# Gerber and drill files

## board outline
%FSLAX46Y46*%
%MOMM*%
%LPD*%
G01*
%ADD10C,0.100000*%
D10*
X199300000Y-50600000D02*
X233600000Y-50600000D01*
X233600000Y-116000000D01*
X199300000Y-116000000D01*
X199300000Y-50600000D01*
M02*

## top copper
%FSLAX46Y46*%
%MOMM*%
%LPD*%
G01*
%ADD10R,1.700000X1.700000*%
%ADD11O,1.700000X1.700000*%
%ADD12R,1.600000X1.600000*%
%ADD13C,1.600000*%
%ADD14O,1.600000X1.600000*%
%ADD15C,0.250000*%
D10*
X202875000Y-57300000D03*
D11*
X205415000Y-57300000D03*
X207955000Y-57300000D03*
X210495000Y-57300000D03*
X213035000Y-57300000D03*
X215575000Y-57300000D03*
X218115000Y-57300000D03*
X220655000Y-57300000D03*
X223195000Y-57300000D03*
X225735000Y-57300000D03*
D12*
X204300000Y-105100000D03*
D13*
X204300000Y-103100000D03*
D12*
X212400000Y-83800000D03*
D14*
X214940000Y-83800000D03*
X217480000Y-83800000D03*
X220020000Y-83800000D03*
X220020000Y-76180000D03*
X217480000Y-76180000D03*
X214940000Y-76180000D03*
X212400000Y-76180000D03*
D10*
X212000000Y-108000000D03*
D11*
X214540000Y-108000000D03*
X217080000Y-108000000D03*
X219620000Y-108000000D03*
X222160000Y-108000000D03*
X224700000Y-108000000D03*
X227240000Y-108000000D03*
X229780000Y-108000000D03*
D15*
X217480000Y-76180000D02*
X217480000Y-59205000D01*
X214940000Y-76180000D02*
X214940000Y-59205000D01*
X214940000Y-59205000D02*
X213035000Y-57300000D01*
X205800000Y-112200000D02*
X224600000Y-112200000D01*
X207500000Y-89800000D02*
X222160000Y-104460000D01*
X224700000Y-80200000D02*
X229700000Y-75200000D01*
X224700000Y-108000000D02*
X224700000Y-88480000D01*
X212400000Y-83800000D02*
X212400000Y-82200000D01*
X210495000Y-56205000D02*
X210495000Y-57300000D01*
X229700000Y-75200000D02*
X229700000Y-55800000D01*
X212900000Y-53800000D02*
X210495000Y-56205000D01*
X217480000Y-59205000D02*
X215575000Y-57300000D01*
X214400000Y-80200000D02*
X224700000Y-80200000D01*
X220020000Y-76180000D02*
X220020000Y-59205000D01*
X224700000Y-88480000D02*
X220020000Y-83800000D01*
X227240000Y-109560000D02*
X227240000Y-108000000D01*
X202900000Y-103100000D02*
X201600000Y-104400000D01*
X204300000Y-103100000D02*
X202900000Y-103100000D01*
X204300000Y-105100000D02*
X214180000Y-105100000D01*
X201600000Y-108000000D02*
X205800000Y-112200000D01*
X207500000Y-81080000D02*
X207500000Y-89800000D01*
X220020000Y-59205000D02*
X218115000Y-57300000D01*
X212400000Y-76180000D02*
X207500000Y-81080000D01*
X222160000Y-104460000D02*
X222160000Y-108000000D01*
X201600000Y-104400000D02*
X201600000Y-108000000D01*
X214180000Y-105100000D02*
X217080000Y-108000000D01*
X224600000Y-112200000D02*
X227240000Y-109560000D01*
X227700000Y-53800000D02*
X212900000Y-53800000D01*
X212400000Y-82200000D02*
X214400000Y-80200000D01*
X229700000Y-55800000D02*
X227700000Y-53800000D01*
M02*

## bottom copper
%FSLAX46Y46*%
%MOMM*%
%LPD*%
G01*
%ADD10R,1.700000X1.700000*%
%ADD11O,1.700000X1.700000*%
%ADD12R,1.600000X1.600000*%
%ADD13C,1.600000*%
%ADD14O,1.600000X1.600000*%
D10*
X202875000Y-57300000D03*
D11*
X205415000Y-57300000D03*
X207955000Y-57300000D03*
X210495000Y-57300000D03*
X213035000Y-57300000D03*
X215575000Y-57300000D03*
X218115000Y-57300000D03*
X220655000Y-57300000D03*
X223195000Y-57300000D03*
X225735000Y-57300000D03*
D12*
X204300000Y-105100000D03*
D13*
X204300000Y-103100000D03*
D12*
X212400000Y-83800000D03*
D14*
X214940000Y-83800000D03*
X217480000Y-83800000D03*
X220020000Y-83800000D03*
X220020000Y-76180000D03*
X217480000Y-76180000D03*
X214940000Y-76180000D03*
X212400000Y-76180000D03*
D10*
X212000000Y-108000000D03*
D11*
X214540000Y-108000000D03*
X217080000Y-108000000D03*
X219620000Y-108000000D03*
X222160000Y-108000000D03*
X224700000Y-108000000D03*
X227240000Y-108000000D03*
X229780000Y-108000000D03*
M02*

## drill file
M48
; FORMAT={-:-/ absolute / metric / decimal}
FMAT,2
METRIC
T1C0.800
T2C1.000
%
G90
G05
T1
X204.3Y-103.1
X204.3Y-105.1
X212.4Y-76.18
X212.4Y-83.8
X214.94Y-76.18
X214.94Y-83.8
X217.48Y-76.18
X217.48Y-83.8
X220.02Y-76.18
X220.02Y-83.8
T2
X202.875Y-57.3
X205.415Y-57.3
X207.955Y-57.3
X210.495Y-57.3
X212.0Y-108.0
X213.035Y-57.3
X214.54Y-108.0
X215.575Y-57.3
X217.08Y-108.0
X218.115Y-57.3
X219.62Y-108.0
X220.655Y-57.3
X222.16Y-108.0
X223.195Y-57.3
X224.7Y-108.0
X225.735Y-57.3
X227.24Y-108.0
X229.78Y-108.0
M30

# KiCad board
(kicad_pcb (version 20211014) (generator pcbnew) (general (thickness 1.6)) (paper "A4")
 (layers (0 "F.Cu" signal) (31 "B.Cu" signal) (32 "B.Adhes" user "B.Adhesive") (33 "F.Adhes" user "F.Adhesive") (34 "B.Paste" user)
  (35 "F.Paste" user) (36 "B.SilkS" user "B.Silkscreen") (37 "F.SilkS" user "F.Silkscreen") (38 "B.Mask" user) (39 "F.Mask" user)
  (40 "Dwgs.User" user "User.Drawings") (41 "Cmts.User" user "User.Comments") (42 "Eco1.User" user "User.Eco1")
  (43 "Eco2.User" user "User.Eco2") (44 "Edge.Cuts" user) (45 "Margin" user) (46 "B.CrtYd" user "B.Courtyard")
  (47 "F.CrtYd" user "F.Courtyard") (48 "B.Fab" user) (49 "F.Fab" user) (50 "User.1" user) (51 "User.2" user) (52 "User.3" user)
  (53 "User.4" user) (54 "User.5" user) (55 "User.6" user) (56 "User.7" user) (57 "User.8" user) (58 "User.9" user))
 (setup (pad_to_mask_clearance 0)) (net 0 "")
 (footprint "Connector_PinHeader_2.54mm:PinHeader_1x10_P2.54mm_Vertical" (layer "F.Cu") (at 202.875 57.3 90)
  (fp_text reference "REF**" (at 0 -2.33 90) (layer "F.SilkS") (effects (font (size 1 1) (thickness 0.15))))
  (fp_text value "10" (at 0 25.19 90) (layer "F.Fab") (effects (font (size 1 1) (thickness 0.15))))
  (pad "1" thru_hole rect (at 0 0 90) (size 1.7 1.7) (drill 1) (layers *.Cu *.Mask))
  (pad "2" thru_hole oval (at 0 2.54 90) (size 1.7 1.7) (drill 1) (layers *.Cu *.Mask))
  (pad "3" thru_hole oval (at 0 5.08 90) (size 1.7 1.7) (drill 1) (layers *.Cu *.Mask))
  (pad "4" thru_hole oval (at 0 7.62 90) (size 1.7 1.7) (drill 1) (layers *.Cu *.Mask))
  (pad "5" thru_hole oval (at 0 10.16 90) (size 1.7 1.7) (drill 1) (layers *.Cu *.Mask))
  (pad "6" thru_hole oval (at 0 12.7 90) (size 1.7 1.7) (drill 1) (layers *.Cu *.Mask))
  (pad "7" thru_hole oval (at 0 15.24 90) (size 1.7 1.7) (drill 1) (layers *.Cu *.Mask))
  (pad "8" thru_hole oval (at 0 17.78 90) (size 1.7 1.7) (drill 1) (layers *.Cu *.Mask))
  (pad "9" thru_hole oval (at 0 20.32 90) (size 1.7 1.7) (drill 1) (layers *.Cu *.Mask))
  (pad "10" thru_hole oval (at 0 22.86 90) (size 1.7 1.7) (drill 1) (layers *.Cu *.Mask)))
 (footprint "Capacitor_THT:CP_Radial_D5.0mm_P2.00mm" (layer "F.Cu") (at 204.3 105.1 90)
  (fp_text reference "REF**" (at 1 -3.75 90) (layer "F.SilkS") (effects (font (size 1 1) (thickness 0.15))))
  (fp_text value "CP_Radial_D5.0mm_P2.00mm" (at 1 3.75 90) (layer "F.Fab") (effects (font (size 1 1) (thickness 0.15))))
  (pad "1" thru_hole rect (at 0 0 90) (size 1.6 1.6) (drill 0.8) (layers *.Cu *.Mask))
  (pad "2" thru_hole circle (at 2 0 90) (size 1.6 1.6) (drill 0.8) (layers *.Cu *.Mask)))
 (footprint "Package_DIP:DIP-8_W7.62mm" (layer "F.Cu") (at 212.4 83.8 90)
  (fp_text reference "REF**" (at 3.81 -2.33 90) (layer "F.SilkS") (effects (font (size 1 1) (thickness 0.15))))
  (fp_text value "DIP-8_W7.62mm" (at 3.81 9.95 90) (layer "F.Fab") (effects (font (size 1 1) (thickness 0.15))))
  (pad "1" thru_hole rect (at 0 0 90) (size 1.6 1.6) (drill 0.8) (layers *.Cu *.Mask))
  (pad "2" thru_hole oval (at 0 2.54 90) (size 1.6 1.6) (drill 0.8) (layers *.Cu *.Mask))
  (pad "3" thru_hole oval (at 0 5.08 90) (size 1.6 1.6) (drill 0.8) (layers *.Cu *.Mask))
  (pad "4" thru_hole oval (at 0 7.62 90) (size 1.6 1.6) (drill 0.8) (layers *.Cu *.Mask))
  (pad "5" thru_hole oval (at 7.62 7.62 90) (size 1.6 1.6) (drill 0.8) (layers *.Cu *.Mask))
  (pad "6" thru_hole oval (at 7.62 5.08 90) (size 1.6 1.6) (drill 0.8) (layers *.Cu *.Mask))
  (pad "7" thru_hole oval (at 7.62 2.54 90) (size 1.6 1.6) (drill 0.8) (layers *.Cu *.Mask))
  (pad "8" thru_hole oval (at 7.62 0 90) (size 1.6 1.6) (drill 0.8) (layers *.Cu *.Mask)))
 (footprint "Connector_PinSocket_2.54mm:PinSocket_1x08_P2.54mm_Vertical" (layer "F.Cu") (at 212 108 90)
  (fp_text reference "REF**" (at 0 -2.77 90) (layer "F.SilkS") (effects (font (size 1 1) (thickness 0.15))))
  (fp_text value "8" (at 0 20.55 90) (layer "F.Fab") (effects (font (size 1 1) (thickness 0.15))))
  (pad "1" thru_hole rect (at 0 0 90) (size 1.7 1.7) (drill 1) (layers *.Cu *.Mask))
  (pad "2" thru_hole oval (at 0 2.54 90) (size 1.7 1.7) (drill 1) (layers *.Cu *.Mask))
  (pad "3" thru_hole oval (at 0 5.08 90) (size 1.7 1.7) (drill 1) (layers *.Cu *.Mask))
  (pad "4" thru_hole oval (at 0 7.62 90) (size 1.7 1.7) (drill 1) (layers *.Cu *.Mask))
  (pad "5" thru_hole oval (at 0 10.16 90) (size 1.7 1.7) (drill 1) (layers *.Cu *.Mask))
  (pad "6" thru_hole oval (at 0 12.7 90) (size 1.7 1.7) (drill 1) (layers *.Cu *.Mask))
  (pad "7" thru_hole oval (at 0 15.24 90) (size 1.7 1.7) (drill 1) (layers *.Cu *.Mask))
  (pad "8" thru_hole oval (at 0 17.78 90) (size 1.7 1.7) (drill 1) (layers *.Cu *.Mask)))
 (gr_rect (start 199.3 50.6) (end 233.6 116) (layer "Edge.Cuts") (width 0.1) (fill none))
 (segment (start 217.48 76.18) (end 217.48 59.205) (width 0.25) (layer "F.Cu") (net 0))
 (segment (start 214.94 76.18) (end 214.94 59.205) (width 0.25) (layer "F.Cu") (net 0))
 (segment (start 214.94 59.205) (end 213.035 57.3) (width 0.25) (layer "F.Cu") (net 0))
 (segment (start 205.8 112.2) (end 224.6 112.2) (width 0.25) (layer "F.Cu") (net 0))
 (segment (start 207.5 89.8) (end 222.16 104.46) (width 0.25) (layer "F.Cu") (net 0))
 (segment (start 224.7 80.2) (end 229.7 75.2) (width 0.25) (layer "F.Cu") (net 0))
 (segment (start 224.7 108) (end 224.7 88.48) (width 0.25) (layer "F.Cu") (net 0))
 (segment (start 212.4 83.8) (end 212.4 82.2) (width 0.25) (layer "F.Cu") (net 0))
 (segment (start 210.495 56.205) (end 210.495 57.3) (width 0.25) (layer "F.Cu") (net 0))
 (segment (start 229.7 75.2) (end 229.7 55.8) (width 0.25) (layer "F.Cu") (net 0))
 (segment (start 212.9 53.8) (end 210.495 56.205) (width 0.25) (layer "F.Cu") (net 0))
 (segment (start 217.48 59.205) (end 215.575 57.3) (width 0.25) (layer "F.Cu") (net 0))
 (segment (start 214.4 80.2) (end 224.7 80.2) (width 0.25) (layer "F.Cu") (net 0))
 (segment (start 220.02 76.18) (end 220.02 59.205) (width 0.25) (layer "F.Cu") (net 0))
 (segment (start 224.7 88.48) (end 220.02 83.8) (width 0.25) (layer "F.Cu") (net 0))
 (segment (start 227.24 109.56) (end 227.24 108) (width 0.25) (layer "F.Cu") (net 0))
 (segment (start 202.9 103.1) (end 201.6 104.4) (width 0.25) (layer "F.Cu") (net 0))
 (segment (start 204.3 103.1) (end 202.9 103.1) (width 0.25) (layer "F.Cu") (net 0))
 (segment (start 204.3 105.1) (end 214.18 105.1) (width 0.25) (layer "F.Cu") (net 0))
 (segment (start 201.6 108) (end 205.8 112.2) (width 0.25) (layer "F.Cu") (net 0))
 (segment (start 207.5 81.08) (end 207.5 89.8) (width 0.25) (layer "F.Cu") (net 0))
 (segment (start 220.02 59.205) (end 218.115 57.3) (width 0.25) (layer "F.Cu") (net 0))
 (segment (start 212.4 76.18) (end 207.5 81.08) (width 0.25) (layer "F.Cu") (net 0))
 (segment (start 222.16 104.46) (end 222.16 108) (width 0.25) (layer "F.Cu") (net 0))
 (segment (start 201.6 104.4) (end 201.6 108) (width 0.25) (layer "F.Cu") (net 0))
 (segment (start 214.18 105.1) (end 217.08 108) (width 0.25) (layer "F.Cu") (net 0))
 (segment (start 224.6 112.2) (end 227.24 109.56) (width 0.25) (layer "F.Cu") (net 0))
 (segment (start 227.7 53.8) (end 212.9 53.8) (width 0.25) (layer "F.Cu") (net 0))
 (segment (start 212.4 82.2) (end 214.4 80.2) (width 0.25) (layer "F.Cu") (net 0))
 (segment (start 229.7 55.8) (end 227.7 53.8) (width 0.25) (layer "F.Cu") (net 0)))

